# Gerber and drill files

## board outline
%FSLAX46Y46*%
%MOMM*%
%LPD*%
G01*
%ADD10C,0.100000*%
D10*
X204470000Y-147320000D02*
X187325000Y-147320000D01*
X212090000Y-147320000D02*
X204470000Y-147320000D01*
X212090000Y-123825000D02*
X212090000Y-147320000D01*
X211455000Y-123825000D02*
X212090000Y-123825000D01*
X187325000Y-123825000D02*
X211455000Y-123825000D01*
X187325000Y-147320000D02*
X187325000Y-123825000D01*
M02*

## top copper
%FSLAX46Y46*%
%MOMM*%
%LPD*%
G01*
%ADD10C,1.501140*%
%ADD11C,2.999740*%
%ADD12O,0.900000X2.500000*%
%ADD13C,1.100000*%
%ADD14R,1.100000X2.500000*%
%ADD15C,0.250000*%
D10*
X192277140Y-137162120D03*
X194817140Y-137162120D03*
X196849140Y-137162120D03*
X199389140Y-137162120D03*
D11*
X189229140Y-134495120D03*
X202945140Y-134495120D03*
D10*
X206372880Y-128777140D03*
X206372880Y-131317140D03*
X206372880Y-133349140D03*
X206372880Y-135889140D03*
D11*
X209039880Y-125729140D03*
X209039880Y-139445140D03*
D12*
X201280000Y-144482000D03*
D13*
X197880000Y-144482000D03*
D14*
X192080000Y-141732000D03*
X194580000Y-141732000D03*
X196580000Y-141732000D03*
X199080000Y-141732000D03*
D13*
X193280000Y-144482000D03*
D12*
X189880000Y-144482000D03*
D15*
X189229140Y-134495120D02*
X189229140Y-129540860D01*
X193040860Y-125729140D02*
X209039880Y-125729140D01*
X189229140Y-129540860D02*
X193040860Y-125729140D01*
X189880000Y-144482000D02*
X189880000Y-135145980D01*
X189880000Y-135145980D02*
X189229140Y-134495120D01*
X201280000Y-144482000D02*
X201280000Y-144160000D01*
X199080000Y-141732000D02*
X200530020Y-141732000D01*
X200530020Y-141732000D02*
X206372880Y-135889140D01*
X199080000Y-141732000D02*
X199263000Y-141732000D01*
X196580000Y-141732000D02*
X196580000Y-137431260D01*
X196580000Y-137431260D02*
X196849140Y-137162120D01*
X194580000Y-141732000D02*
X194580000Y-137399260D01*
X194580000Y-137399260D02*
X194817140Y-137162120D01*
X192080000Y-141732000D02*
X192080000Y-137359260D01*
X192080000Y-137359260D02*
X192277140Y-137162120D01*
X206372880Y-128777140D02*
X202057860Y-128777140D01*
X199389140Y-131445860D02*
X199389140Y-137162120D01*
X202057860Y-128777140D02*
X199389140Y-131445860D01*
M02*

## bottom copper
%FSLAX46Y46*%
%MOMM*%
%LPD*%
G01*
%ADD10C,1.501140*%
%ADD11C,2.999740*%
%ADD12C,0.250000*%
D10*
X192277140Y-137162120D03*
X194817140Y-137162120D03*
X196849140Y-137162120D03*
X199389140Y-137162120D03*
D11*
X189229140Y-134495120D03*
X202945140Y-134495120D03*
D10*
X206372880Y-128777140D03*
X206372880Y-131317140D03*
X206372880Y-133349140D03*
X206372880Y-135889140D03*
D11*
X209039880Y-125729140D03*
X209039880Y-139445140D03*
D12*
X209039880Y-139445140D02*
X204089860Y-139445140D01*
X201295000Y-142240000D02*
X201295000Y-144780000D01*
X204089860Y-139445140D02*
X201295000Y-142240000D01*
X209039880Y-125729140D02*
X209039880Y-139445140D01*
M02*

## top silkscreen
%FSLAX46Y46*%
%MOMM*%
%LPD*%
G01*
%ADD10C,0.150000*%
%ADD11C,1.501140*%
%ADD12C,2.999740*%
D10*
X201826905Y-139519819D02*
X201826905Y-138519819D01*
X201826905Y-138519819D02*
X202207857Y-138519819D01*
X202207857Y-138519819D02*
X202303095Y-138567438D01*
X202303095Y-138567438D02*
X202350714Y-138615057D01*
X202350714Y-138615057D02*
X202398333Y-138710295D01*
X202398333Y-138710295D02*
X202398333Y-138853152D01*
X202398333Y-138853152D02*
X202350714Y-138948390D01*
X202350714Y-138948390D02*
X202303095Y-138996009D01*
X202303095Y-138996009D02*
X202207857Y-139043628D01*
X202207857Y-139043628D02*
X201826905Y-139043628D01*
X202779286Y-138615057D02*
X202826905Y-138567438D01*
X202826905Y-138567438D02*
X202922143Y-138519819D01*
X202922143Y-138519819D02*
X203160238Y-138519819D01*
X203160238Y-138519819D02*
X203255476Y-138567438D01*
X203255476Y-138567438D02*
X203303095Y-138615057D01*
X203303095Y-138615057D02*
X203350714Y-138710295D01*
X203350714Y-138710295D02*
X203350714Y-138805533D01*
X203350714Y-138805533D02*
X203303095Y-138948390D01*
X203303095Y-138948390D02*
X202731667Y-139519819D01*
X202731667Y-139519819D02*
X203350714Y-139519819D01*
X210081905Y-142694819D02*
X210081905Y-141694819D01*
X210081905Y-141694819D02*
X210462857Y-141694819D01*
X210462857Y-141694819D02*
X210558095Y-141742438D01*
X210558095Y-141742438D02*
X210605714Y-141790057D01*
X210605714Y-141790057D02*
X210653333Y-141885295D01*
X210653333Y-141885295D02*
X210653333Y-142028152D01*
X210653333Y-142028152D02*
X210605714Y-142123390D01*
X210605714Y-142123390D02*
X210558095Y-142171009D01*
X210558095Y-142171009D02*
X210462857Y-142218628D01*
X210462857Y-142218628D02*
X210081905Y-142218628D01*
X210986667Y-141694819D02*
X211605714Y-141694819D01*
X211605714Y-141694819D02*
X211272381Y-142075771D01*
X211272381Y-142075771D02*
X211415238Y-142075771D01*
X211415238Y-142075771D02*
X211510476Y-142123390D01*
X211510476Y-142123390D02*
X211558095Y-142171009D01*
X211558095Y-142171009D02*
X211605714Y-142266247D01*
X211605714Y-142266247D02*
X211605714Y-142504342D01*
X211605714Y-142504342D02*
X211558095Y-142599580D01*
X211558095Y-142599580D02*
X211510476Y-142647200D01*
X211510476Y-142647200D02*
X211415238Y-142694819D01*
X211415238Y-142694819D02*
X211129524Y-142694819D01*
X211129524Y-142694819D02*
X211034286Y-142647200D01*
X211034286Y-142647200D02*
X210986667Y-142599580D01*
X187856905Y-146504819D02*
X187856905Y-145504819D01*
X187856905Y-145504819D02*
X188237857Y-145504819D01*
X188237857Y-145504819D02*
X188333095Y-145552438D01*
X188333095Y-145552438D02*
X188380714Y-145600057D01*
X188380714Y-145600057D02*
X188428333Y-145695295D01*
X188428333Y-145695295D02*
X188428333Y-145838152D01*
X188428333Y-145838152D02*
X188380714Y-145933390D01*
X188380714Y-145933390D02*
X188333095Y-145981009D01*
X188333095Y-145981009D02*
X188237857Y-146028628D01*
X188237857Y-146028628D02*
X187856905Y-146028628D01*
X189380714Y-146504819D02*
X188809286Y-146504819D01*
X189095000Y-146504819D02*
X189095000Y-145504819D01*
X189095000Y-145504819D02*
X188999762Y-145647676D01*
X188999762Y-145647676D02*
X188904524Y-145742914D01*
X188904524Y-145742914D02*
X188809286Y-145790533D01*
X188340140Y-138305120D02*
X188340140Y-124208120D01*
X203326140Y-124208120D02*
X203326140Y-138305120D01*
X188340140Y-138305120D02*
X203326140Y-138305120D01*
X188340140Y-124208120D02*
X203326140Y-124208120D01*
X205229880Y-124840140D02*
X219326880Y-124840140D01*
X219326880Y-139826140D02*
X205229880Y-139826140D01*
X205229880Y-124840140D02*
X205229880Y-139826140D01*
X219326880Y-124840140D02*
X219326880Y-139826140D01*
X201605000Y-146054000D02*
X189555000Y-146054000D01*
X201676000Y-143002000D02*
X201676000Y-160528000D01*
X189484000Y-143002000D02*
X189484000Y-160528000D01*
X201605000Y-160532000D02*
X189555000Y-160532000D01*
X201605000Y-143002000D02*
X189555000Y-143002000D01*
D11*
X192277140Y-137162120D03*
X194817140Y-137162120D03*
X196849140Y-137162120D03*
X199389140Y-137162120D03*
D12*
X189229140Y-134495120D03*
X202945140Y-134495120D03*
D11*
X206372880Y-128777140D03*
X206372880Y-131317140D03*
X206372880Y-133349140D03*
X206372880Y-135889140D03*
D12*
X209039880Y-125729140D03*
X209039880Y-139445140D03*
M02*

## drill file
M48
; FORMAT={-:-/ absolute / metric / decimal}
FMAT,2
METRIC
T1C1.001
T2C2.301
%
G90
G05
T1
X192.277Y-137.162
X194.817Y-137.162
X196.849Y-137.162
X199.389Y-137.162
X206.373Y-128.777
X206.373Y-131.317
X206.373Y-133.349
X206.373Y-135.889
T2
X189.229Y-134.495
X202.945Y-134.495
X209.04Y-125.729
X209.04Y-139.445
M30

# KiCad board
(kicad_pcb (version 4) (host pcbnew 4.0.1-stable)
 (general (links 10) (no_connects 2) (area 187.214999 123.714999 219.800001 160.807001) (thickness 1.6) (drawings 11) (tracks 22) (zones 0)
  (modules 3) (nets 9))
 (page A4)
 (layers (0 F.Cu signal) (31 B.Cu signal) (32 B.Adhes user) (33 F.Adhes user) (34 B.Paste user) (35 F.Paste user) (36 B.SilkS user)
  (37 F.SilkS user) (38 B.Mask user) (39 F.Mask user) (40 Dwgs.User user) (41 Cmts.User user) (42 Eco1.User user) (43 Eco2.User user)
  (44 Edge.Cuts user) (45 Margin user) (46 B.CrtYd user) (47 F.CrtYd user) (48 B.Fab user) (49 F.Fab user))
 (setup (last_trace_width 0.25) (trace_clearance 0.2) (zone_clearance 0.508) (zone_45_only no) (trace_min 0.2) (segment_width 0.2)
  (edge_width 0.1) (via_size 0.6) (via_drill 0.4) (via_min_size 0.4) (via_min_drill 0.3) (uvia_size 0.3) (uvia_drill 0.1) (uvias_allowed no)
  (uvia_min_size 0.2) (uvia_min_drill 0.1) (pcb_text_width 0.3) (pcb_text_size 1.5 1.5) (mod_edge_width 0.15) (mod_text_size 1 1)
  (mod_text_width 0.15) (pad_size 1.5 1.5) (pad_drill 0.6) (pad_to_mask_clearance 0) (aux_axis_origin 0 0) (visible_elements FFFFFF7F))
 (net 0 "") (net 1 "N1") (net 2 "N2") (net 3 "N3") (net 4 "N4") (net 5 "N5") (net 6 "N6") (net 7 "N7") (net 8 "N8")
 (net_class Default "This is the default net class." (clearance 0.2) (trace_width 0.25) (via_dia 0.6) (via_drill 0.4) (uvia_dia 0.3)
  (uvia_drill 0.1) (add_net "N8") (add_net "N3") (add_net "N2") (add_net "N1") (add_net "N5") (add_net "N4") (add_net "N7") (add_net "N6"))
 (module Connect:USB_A (layer F.Cu) (at 199.39 137.16 180)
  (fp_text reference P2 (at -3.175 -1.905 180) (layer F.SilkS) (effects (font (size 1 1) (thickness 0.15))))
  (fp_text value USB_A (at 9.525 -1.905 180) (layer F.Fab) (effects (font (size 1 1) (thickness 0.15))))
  (fp_line (start 11.04986 -1.14512) (end 11.04986 12.95188) (layer F.SilkS) (width 0.15))
  (fp_line (start -3.93614 12.95188) (end -3.93614 -1.14512) (layer F.SilkS) (width 0.15))
  (fp_line (start 11.04986 -1.14512) (end -3.93614 -1.14512) (layer F.SilkS) (width 0.15))
  (fp_line (start 11.04986 12.95188) (end -3.93614 12.95188) (layer F.SilkS) (width 0.15))
  (pad 4 thru_hole circle (at 7.11286 -0.00212 90) (size 1.50114 1.50114) (drill 1.00076) (layers *.Cu *.Mask F.SilkS) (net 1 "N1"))
  (pad 3 thru_hole circle (at 4.57286 -0.00212 90) (size 1.50114 1.50114) (drill 1.00076) (layers *.Cu *.Mask F.SilkS) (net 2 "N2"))
  (pad 2 thru_hole circle (at 2.54086 -0.00212 90) (size 1.50114 1.50114) (drill 1.00076) (layers *.Cu *.Mask F.SilkS) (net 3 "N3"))
  (pad 1 thru_hole circle (at 0.00086 -0.00212 90) (size 1.50114 1.50114) (drill 1.00076) (layers *.Cu *.Mask F.SilkS) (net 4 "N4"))
  (pad 5 thru_hole circle (at 10.16086 2.66488 90) (size 2.99974 2.99974) (drill 2.30124) (layers *.Cu *.Mask F.SilkS) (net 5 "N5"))
  (pad 5 thru_hole circle (at -3.55514 2.66488 90) (size 2.99974 2.99974) (drill 2.30124) (layers *.Cu *.Mask F.SilkS) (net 5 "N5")))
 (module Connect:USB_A (layer F.Cu) (at 206.375 135.89 90)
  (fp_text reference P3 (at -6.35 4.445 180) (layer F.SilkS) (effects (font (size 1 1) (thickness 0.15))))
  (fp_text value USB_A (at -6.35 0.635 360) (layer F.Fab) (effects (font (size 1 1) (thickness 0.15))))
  (fp_line (start 11.04986 -1.14512) (end 11.04986 12.95188) (layer F.SilkS) (width 0.15))
  (fp_line (start -3.93614 12.95188) (end -3.93614 -1.14512) (layer F.SilkS) (width 0.15))
  (fp_line (start 11.04986 -1.14512) (end -3.93614 -1.14512) (layer F.SilkS) (width 0.15))
  (fp_line (start 11.04986 12.95188) (end -3.93614 12.95188) (layer F.SilkS) (width 0.15))
  (pad 4 thru_hole circle (at 7.11286 -0.00212) (size 1.50114 1.50114) (drill 1.00076) (layers *.Cu *.Mask F.SilkS) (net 4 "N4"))
  (pad 3 thru_hole circle (at 4.57286 -0.00212) (size 1.50114 1.50114) (drill 1.00076) (layers *.Cu *.Mask F.SilkS) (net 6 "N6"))
  (pad 2 thru_hole circle (at 2.54086 -0.00212) (size 1.50114 1.50114) (drill 1.00076) (layers *.Cu *.Mask F.SilkS) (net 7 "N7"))
  (pad 1 thru_hole circle (at 0.00086 -0.00212) (size 1.50114 1.50114) (drill 1.00076) (layers *.Cu *.Mask F.SilkS) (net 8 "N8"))
  (pad 5 thru_hole circle (at 10.16086 2.66488) (size 2.99974 2.99974) (drill 2.30124) (layers *.Cu *.Mask F.SilkS) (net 5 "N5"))
  (pad 5 thru_hole circle (at -3.55514 2.66488) (size 2.99974 2.99974) (drill 2.30124) (layers *.Cu *.Mask F.SilkS) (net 5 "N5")))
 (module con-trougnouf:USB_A (layer F.Cu) (at 195.58 146.05)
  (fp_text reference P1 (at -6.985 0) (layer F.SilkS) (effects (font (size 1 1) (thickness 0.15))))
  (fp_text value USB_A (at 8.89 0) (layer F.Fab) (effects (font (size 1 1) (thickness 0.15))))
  (fp_line (start 6.025 0.004) (end -6.025 0.004) (layer F.SilkS) (width 0.15))
  (fp_line (start 6.096 -3.048) (end 6.096 14.478) (layer F.SilkS) (width 0.15))
  (fp_line (start -6.096 -3.048) (end -6.096 14.478) (layer F.SilkS) (width 0.15))
  (fp_line (start 6.025 14.482) (end -6.025 14.482) (layer F.SilkS) (width 0.15))
  (fp_line (start 6.025 -3.048) (end -6.025 -3.048) (layer F.SilkS) (width 0.15))
  (pad 5 smd oval (at 5.7 -1.568) (size 0.9 2.5) (layers F.Cu F.Paste F.Mask) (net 5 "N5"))
  (pad "" smd circle (at 2.3 -1.568) (size 1.1 1.1) (layers F.Cu F.Paste F.Mask))
  (pad 4 smd rect (at -3.5 -4.318) (size 1.1 2.5) (layers F.Cu F.Paste F.Mask) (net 1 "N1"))
  (pad 3 smd rect (at -1 -4.318) (size 1.1 2.5) (layers F.Cu F.Paste F.Mask) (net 2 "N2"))
  (pad 2 smd rect (at 1 -4.318) (size 1.1 2.5) (layers F.Cu F.Paste F.Mask) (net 3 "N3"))
  (pad 1 smd rect (at 3.5 -4.318) (size 1.1 2.5) (layers F.Cu F.Paste F.Mask) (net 8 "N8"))
  (pad "" smd circle (at -2.3 -1.568) (size 1.1 1.1) (layers F.Cu F.Paste F.Mask))
  (pad 5 smd oval (at -5.7 -1.568) (size 0.9 2.5) (layers F.Cu F.Paste F.Mask) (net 5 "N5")))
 (gr_line (start 204.47 147.32) (end 187.325 147.32) (angle 90) (layer Edge.Cuts) (width 0.1))
 (gr_line (start 212.09 147.32) (end 204.47 147.32) (angle 90) (layer Edge.Cuts) (width 0.1))
 (gr_line (start 212.09 123.825) (end 212.09 147.32) (angle 90) (layer Edge.Cuts) (width 0.1))
 (gr_line (start 211.455 123.825) (end 212.09 123.825) (angle 90) (layer Edge.Cuts) (width 0.1))
 (gr_line (start 187.325 123.825) (end 211.455 123.825) (angle 90) (layer Edge.Cuts) (width 0.1))
 (gr_line (start 187.325 147.32) (end 187.325 123.825) (angle 90) (layer Edge.Cuts) (width 0.1))
 (segment (start 209.03988 139.44514) (end 204.08986 139.44514) (width 0.25) (layer B.Cu) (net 5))
 (segment (start 201.295 142.24) (end 201.295 144.78) (width 0.25) (layer B.Cu) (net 5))
 (segment (start 204.08986 139.44514) (end 201.295 142.24) (width 0.25) (layer B.Cu) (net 5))
 (segment (start 209.03988 125.72914) (end 209.03988 139.44514) (width 0.25) (layer B.Cu) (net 5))
 (segment (start 189.22914 134.49512) (end 189.22914 129.54086) (width 0.25) (layer F.Cu) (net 5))
 (segment (start 193.04086 125.72914) (end 209.03988 125.72914) (width 0.25) (layer F.Cu) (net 5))
 (segment (start 189.22914 129.54086) (end 193.04086 125.72914) (width 0.25) (layer F.Cu) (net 5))
 (segment (start 189.88 144.482) (end 189.88 135.14598) (width 0.25) (layer F.Cu) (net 5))
 (segment (start 189.88 135.14598) (end 189.22914 134.49512) (width 0.25) (layer F.Cu) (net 5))
 (segment (start 201.28 144.482) (end 201.28 144.16) (width 0.25) (layer F.Cu) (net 5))
 (segment (start 199.08 141.732) (end 200.53002 141.732) (width 0.25) (layer F.Cu) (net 8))
 (segment (start 200.53002 141.732) (end 206.37288 135.88914) (width 0.25) (layer F.Cu) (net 8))
 (segment (start 199.08 141.732) (end 199.263 141.732) (width 0.25) (layer F.Cu) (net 8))
 (segment (start 196.58 141.732) (end 196.58 137.43126) (width 0.25) (layer F.Cu) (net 3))
 (segment (start 196.58 137.43126) (end 196.84914 137.16212) (width 0.25) (layer F.Cu) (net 3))
 (segment (start 194.58 141.732) (end 194.58 137.39926) (width 0.25) (layer F.Cu) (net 2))
 (segment (start 194.58 137.39926) (end 194.81714 137.16212) (width 0.25) (layer F.Cu) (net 2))
 (segment (start 192.08 141.732) (end 192.08 137.35926) (width 0.25) (layer F.Cu) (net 1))
 (segment (start 192.08 137.35926) (end 192.27714 137.16212) (width 0.25) (layer F.Cu) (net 1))
 (segment (start 206.37288 128.77714) (end 202.05786 128.77714) (width 0.25) (layer F.Cu) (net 4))
 (segment (start 199.38914 131.44586) (end 199.38914 137.16212) (width 0.25) (layer F.Cu) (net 4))
 (segment (start 202.05786 128.77714) (end 199.38914 131.44586) (width 0.25) (layer F.Cu) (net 4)))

